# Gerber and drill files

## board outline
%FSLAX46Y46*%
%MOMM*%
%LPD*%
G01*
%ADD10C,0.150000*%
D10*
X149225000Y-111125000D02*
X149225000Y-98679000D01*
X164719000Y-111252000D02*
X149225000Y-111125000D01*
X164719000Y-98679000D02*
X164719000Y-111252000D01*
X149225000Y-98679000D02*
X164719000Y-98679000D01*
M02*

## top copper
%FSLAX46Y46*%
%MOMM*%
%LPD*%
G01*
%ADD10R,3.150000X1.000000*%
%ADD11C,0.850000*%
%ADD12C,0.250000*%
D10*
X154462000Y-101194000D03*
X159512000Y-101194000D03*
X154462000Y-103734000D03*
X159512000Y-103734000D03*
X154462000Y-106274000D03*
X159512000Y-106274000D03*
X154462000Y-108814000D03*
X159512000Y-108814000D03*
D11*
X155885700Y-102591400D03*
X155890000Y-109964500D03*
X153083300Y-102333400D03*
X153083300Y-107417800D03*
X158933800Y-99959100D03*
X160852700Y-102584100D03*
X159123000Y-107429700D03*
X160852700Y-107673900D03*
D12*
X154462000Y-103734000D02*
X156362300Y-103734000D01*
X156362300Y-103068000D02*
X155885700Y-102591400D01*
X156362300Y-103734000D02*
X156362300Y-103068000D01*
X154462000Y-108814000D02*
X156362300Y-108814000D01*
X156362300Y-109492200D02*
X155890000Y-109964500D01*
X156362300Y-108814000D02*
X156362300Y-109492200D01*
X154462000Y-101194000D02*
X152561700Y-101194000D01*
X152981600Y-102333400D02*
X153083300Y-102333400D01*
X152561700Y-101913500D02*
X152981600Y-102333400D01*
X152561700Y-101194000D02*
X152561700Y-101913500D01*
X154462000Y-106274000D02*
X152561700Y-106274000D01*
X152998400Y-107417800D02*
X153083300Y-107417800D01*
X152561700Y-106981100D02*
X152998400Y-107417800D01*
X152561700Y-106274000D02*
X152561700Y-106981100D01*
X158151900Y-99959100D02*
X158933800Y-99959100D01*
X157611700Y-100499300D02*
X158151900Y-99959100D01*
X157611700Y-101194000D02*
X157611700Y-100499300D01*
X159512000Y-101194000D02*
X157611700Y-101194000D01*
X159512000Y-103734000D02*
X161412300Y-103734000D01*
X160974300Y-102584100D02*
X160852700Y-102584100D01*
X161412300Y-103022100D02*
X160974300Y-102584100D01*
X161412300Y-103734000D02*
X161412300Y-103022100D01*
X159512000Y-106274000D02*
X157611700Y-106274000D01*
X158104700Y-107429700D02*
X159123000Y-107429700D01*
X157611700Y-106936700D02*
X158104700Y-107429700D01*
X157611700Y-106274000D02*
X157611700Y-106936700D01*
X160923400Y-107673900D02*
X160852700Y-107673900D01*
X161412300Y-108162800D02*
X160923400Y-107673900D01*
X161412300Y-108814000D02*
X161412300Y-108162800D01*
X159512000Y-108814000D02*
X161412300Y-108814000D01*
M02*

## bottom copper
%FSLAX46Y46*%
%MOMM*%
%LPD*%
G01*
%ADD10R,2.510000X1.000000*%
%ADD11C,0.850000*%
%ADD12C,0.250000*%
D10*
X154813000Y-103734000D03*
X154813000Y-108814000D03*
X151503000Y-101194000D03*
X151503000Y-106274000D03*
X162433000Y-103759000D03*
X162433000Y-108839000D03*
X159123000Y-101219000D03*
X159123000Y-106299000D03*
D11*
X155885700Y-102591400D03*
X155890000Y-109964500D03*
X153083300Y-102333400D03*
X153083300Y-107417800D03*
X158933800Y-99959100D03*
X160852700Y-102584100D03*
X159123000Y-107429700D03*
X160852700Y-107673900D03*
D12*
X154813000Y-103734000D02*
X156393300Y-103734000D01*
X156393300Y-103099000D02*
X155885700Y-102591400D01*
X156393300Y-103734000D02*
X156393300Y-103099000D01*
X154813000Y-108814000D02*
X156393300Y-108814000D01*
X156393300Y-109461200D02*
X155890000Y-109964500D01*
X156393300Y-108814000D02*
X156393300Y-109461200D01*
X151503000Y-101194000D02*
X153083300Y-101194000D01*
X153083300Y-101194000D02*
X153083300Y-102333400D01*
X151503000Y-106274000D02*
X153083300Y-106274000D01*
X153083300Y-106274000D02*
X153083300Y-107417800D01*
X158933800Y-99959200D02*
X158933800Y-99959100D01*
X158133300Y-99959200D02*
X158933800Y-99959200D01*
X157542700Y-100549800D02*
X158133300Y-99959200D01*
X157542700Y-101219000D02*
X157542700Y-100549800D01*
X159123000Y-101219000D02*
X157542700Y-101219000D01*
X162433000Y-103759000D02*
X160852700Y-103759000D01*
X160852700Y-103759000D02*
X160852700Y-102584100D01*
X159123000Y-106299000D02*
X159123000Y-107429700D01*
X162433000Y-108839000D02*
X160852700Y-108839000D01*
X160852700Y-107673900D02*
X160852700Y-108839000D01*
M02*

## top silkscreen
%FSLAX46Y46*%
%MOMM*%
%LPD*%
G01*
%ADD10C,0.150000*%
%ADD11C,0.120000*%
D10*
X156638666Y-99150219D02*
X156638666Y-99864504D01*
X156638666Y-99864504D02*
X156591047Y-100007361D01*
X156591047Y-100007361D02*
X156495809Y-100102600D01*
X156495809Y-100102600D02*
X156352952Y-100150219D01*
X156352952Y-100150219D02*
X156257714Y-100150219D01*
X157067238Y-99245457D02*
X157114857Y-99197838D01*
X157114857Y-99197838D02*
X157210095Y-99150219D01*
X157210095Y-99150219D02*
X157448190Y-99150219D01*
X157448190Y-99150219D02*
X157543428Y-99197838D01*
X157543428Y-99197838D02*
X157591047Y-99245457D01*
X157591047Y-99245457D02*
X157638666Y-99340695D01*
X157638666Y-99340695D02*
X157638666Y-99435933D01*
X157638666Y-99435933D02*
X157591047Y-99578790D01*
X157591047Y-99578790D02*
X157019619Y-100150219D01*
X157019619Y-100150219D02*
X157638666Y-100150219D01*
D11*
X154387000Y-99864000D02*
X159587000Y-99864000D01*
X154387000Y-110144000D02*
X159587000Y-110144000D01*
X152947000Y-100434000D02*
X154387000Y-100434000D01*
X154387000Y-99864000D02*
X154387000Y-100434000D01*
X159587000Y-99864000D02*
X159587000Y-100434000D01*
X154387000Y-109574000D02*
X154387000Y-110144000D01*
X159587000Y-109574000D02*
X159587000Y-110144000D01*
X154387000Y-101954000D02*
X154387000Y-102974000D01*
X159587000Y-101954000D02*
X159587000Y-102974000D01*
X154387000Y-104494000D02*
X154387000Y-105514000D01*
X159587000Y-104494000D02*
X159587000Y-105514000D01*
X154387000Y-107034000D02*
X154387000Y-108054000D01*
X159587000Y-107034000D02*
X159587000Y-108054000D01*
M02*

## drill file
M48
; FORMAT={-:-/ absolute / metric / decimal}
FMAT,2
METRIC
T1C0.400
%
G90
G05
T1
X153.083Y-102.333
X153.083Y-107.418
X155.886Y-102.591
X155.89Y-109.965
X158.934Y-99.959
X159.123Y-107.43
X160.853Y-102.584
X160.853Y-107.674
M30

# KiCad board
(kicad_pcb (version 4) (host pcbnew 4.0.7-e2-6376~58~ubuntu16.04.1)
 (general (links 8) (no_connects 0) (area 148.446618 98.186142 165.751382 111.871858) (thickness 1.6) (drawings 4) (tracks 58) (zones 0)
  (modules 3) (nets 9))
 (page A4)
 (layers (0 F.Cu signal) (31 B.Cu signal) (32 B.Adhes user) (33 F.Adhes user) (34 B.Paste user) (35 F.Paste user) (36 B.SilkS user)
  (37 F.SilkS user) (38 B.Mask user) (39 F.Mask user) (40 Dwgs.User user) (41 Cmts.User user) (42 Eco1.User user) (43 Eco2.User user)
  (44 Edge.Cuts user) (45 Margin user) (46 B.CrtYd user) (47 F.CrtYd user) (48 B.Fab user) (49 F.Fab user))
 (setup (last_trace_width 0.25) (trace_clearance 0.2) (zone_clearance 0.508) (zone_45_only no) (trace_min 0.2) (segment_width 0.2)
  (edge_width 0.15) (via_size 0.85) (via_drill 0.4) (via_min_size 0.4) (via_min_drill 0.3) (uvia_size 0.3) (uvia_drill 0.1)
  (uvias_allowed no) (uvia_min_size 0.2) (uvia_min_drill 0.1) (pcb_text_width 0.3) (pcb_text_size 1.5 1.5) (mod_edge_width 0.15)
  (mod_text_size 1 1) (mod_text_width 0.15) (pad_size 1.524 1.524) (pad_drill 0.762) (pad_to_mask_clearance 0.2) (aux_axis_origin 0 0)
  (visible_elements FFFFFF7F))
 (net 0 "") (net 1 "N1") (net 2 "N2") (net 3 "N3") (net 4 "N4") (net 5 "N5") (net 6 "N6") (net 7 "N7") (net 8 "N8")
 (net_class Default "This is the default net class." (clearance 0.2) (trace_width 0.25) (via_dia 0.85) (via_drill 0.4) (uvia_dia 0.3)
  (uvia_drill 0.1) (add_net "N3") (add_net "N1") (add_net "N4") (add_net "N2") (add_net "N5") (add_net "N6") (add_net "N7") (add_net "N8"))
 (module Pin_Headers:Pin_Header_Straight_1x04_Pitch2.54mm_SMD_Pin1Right (layer B.Cu) (at 153.158 105.004 180)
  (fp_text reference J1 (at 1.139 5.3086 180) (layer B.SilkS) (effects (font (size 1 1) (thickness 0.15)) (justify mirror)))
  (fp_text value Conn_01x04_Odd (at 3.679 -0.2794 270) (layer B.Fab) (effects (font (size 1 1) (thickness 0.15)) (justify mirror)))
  (pad 2 smd rect (at -1.655 1.27 180) (size 2.51 1) (layers B.Cu B.Paste B.Mask) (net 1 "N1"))
  (pad 4 smd rect (at -1.655 -3.81 180) (size 2.51 1) (layers B.Cu B.Paste B.Mask) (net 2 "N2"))
  (pad 1 smd rect (at 1.655 3.81 180) (size 2.51 1) (layers B.Cu B.Paste B.Mask) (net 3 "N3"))
  (pad 3 smd rect (at 1.655 -1.27 180) (size 2.51 1) (layers B.Cu B.Paste B.Mask) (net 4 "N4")))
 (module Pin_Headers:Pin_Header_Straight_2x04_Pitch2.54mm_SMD (layer F.Cu) (at 156.987 105.004)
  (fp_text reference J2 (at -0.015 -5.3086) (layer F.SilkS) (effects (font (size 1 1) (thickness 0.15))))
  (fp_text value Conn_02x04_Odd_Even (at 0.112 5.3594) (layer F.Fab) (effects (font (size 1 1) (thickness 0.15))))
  (fp_line (start -2.6 -5.14) (end 2.6 -5.14) (layer F.SilkS) (width 0.12))
  (fp_line (start -2.6 5.14) (end 2.6 5.14) (layer F.SilkS) (width 0.12))
  (fp_line (start -4.04 -4.57) (end -2.6 -4.57) (layer F.SilkS) (width 0.12))
  (fp_line (start -2.6 -5.14) (end -2.6 -4.57) (layer F.SilkS) (width 0.12))
  (fp_line (start 2.6 -5.14) (end 2.6 -4.57) (layer F.SilkS) (width 0.12))
  (fp_line (start -2.6 4.57) (end -2.6 5.14) (layer F.SilkS) (width 0.12))
  (fp_line (start 2.6 4.57) (end 2.6 5.14) (layer F.SilkS) (width 0.12))
  (fp_line (start -2.6 -3.05) (end -2.6 -2.03) (layer F.SilkS) (width 0.12))
  (fp_line (start 2.6 -3.05) (end 2.6 -2.03) (layer F.SilkS) (width 0.12))
  (fp_line (start -2.6 -0.51) (end -2.6 0.51) (layer F.SilkS) (width 0.12))
  (fp_line (start 2.6 -0.51) (end 2.6 0.51) (layer F.SilkS) (width 0.12))
  (fp_line (start -2.6 2.03) (end -2.6 3.05) (layer F.SilkS) (width 0.12))
  (fp_line (start 2.6 2.03) (end 2.6 3.05) (layer F.SilkS) (width 0.12))
  (pad 1 smd rect (at -2.525 -3.81) (size 3.15 1) (layers F.Cu F.Paste F.Mask) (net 3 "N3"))
  (pad 2 smd rect (at 2.525 -3.81) (size 3.15 1) (layers F.Cu F.Paste F.Mask) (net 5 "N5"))
  (pad 3 smd rect (at -2.525 -1.27) (size 3.15 1) (layers F.Cu F.Paste F.Mask) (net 1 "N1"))
  (pad 4 smd rect (at 2.525 -1.27) (size 3.15 1) (layers F.Cu F.Paste F.Mask) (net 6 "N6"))
  (pad 5 smd rect (at -2.525 1.27) (size 3.15 1) (layers F.Cu F.Paste F.Mask) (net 4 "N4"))
  (pad 6 smd rect (at 2.525 1.27) (size 3.15 1) (layers F.Cu F.Paste F.Mask) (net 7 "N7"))
  (pad 7 smd rect (at -2.525 3.81) (size 3.15 1) (layers F.Cu F.Paste F.Mask) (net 2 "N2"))
  (pad 8 smd rect (at 2.525 3.81) (size 3.15 1) (layers F.Cu F.Paste F.Mask) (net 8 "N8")))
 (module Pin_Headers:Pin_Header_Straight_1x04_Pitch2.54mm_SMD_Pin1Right (layer B.Cu) (at 160.778 105.029 180)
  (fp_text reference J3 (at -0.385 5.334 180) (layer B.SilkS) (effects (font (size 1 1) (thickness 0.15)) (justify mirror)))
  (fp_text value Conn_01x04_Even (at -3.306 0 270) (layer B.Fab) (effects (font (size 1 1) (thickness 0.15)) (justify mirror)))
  (pad 2 smd rect (at -1.655 1.27 180) (size 2.51 1) (layers B.Cu B.Paste B.Mask) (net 6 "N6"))
  (pad 4 smd rect (at -1.655 -3.81 180) (size 2.51 1) (layers B.Cu B.Paste B.Mask) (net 8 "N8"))
  (pad 1 smd rect (at 1.655 3.81 180) (size 2.51 1) (layers B.Cu B.Paste B.Mask) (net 5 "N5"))
  (pad 3 smd rect (at 1.655 -1.27 180) (size 2.51 1) (layers B.Cu B.Paste B.Mask) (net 7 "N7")))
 (gr_line (start 149.225 111.125) (end 149.225 98.679) (layer Edge.Cuts) (width 0.15))
 (gr_line (start 164.719 111.252) (end 149.225 111.125) (layer Edge.Cuts) (width 0.15))
 (gr_line (start 164.719 98.679) (end 164.719 111.252) (layer Edge.Cuts) (width 0.15))
 (gr_line (start 149.225 98.679) (end 164.719 98.679) (layer Edge.Cuts) (width 0.15))
 (via (at 155.8857 102.5914) (size 0.85) (layers F.Cu B.Cu) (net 1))
 (segment (start 154.462 103.734) (end 156.3623 103.734) (width 0.25) (layer F.Cu) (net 1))
 (segment (start 154.813 103.734) (end 156.3933 103.734) (width 0.25) (layer B.Cu) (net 1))
 (segment (start 156.3933 103.099) (end 155.8857 102.5914) (width 0.25) (layer B.Cu) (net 1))
 (segment (start 156.3933 103.734) (end 156.3933 103.099) (width 0.25) (layer B.Cu) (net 1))
 (segment (start 156.3623 103.068) (end 155.8857 102.5914) (width 0.25) (layer F.Cu) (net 1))
 (segment (start 156.3623 103.734) (end 156.3623 103.068) (width 0.25) (layer F.Cu) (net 1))
 (via (at 155.89 109.9645) (size 0.85) (layers F.Cu B.Cu) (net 2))
 (segment (start 154.462 108.814) (end 156.3623 108.814) (width 0.25) (layer F.Cu) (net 2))
 (segment (start 154.813 108.814) (end 156.3933 108.814) (width 0.25) (layer B.Cu) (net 2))
 (segment (start 156.3933 109.4612) (end 155.89 109.9645) (width 0.25) (layer B.Cu) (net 2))
 (segment (start 156.3933 108.814) (end 156.3933 109.4612) (width 0.25) (layer B.Cu) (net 2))
 (segment (start 156.3623 109.4922) (end 155.89 109.9645) (width 0.25) (layer F.Cu) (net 2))
 (segment (start 156.3623 108.814) (end 156.3623 109.4922) (width 0.25) (layer F.Cu) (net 2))
 (via (at 153.0833 102.3334) (size 0.85) (layers F.Cu B.Cu) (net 3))
 (segment (start 151.503 101.194) (end 153.0833 101.194) (width 0.25) (layer B.Cu) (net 3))
 (segment (start 154.462 101.194) (end 152.5617 101.194) (width 0.25) (layer F.Cu) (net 3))
 (segment (start 153.0833 101.194) (end 153.0833 102.3334) (width 0.25) (layer B.Cu) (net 3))
 (segment (start 152.9816 102.3334) (end 153.0833 102.3334) (width 0.25) (layer F.Cu) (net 3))
 (segment (start 152.5617 101.9135) (end 152.9816 102.3334) (width 0.25) (layer F.Cu) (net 3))
 (segment (start 152.5617 101.194) (end 152.5617 101.9135) (width 0.25) (layer F.Cu) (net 3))
 (via (at 153.0833 107.4178) (size 0.85) (layers F.Cu B.Cu) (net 4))
 (segment (start 151.503 106.274) (end 153.0833 106.274) (width 0.25) (layer B.Cu) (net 4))
 (segment (start 154.462 106.274) (end 152.5617 106.274) (width 0.25) (layer F.Cu) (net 4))
 (segment (start 153.0833 106.274) (end 153.0833 107.4178) (width 0.25) (layer B.Cu) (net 4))
 (segment (start 152.9984 107.4178) (end 153.0833 107.4178) (width 0.25) (layer F.Cu) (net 4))
 (segment (start 152.5617 106.9811) (end 152.9984 107.4178) (width 0.25) (layer F.Cu) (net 4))
 (segment (start 152.5617 106.274) (end 152.5617 106.9811) (width 0.25) (layer F.Cu) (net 4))
 (via (at 158.9338 99.9591) (size 0.85) (layers F.Cu B.Cu) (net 5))
 (segment (start 158.9338 99.9592) (end 158.9338 99.9591) (width 0.25) (layer B.Cu) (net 5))
 (segment (start 158.1333 99.9592) (end 158.9338 99.9592) (width 0.25) (layer B.Cu) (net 5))
 (segment (start 157.5427 100.5498) (end 158.1333 99.9592) (width 0.25) (layer B.Cu) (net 5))
 (segment (start 157.5427 101.219) (end 157.5427 100.5498) (width 0.25) (layer B.Cu) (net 5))
 (segment (start 158.1519 99.9591) (end 158.9338 99.9591) (width 0.25) (layer F.Cu) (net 5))
 (segment (start 157.6117 100.4993) (end 158.1519 99.9591) (width 0.25) (layer F.Cu) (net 5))
 (segment (start 157.6117 101.194) (end 157.6117 100.4993) (width 0.25) (layer F.Cu) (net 5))
 (segment (start 159.512 101.194) (end 157.6117 101.194) (width 0.25) (layer F.Cu) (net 5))
 (segment (start 159.123 101.219) (end 157.5427 101.219) (width 0.25) (layer B.Cu) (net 5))
 (via (at 160.8527 102.5841) (size 0.85) (layers F.Cu B.Cu) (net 6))
 (segment (start 162.433 103.759) (end 160.8527 103.759) (width 0.25) (layer B.Cu) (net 6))
 (segment (start 159.512 103.734) (end 161.4123 103.734) (width 0.25) (layer F.Cu) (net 6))
 (segment (start 160.8527 103.759) (end 160.8527 102.5841) (width 0.25) (layer B.Cu) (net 6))
 (segment (start 160.9743 102.5841) (end 160.8527 102.5841) (width 0.25) (layer F.Cu) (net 6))
 (segment (start 161.4123 103.0221) (end 160.9743 102.5841) (width 0.25) (layer F.Cu) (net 6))
 (segment (start 161.4123 103.734) (end 161.4123 103.0221) (width 0.25) (layer F.Cu) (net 6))
 (via (at 159.123 107.4297) (size 0.85) (layers F.Cu B.Cu) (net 7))
 (segment (start 159.512 106.274) (end 157.6117 106.274) (width 0.25) (layer F.Cu) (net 7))
 (segment (start 159.123 106.299) (end 159.123 107.4297) (width 0.25) (layer B.Cu) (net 7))
 (segment (start 158.1047 107.4297) (end 159.123 107.4297) (width 0.25) (layer F.Cu) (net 7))
 (segment (start 157.6117 106.9367) (end 158.1047 107.4297) (width 0.25) (layer F.Cu) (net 7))
 (segment (start 157.6117 106.274) (end 157.6117 106.9367) (width 0.25) (layer F.Cu) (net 7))
 (via (at 160.8527 107.6739) (size 0.85) (layers F.Cu B.Cu) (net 8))
 (segment (start 162.433 108.839) (end 160.8527 108.839) (width 0.25) (layer B.Cu) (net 8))
 (segment (start 160.8527 107.6739) (end 160.8527 108.839) (width 0.25) (layer B.Cu) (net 8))
 (segment (start 160.9234 107.6739) (end 160.8527 107.6739) (width 0.25) (layer F.Cu) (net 8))
 (segment (start 161.4123 108.1628) (end 160.9234 107.6739) (width 0.25) (layer F.Cu) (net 8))
 (segment (start 161.4123 108.814) (end 161.4123 108.1628) (width 0.25) (layer F.Cu) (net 8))
 (segment (start 159.512 108.814) (end 161.4123 108.814) (width 0.25) (layer F.Cu) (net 8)))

